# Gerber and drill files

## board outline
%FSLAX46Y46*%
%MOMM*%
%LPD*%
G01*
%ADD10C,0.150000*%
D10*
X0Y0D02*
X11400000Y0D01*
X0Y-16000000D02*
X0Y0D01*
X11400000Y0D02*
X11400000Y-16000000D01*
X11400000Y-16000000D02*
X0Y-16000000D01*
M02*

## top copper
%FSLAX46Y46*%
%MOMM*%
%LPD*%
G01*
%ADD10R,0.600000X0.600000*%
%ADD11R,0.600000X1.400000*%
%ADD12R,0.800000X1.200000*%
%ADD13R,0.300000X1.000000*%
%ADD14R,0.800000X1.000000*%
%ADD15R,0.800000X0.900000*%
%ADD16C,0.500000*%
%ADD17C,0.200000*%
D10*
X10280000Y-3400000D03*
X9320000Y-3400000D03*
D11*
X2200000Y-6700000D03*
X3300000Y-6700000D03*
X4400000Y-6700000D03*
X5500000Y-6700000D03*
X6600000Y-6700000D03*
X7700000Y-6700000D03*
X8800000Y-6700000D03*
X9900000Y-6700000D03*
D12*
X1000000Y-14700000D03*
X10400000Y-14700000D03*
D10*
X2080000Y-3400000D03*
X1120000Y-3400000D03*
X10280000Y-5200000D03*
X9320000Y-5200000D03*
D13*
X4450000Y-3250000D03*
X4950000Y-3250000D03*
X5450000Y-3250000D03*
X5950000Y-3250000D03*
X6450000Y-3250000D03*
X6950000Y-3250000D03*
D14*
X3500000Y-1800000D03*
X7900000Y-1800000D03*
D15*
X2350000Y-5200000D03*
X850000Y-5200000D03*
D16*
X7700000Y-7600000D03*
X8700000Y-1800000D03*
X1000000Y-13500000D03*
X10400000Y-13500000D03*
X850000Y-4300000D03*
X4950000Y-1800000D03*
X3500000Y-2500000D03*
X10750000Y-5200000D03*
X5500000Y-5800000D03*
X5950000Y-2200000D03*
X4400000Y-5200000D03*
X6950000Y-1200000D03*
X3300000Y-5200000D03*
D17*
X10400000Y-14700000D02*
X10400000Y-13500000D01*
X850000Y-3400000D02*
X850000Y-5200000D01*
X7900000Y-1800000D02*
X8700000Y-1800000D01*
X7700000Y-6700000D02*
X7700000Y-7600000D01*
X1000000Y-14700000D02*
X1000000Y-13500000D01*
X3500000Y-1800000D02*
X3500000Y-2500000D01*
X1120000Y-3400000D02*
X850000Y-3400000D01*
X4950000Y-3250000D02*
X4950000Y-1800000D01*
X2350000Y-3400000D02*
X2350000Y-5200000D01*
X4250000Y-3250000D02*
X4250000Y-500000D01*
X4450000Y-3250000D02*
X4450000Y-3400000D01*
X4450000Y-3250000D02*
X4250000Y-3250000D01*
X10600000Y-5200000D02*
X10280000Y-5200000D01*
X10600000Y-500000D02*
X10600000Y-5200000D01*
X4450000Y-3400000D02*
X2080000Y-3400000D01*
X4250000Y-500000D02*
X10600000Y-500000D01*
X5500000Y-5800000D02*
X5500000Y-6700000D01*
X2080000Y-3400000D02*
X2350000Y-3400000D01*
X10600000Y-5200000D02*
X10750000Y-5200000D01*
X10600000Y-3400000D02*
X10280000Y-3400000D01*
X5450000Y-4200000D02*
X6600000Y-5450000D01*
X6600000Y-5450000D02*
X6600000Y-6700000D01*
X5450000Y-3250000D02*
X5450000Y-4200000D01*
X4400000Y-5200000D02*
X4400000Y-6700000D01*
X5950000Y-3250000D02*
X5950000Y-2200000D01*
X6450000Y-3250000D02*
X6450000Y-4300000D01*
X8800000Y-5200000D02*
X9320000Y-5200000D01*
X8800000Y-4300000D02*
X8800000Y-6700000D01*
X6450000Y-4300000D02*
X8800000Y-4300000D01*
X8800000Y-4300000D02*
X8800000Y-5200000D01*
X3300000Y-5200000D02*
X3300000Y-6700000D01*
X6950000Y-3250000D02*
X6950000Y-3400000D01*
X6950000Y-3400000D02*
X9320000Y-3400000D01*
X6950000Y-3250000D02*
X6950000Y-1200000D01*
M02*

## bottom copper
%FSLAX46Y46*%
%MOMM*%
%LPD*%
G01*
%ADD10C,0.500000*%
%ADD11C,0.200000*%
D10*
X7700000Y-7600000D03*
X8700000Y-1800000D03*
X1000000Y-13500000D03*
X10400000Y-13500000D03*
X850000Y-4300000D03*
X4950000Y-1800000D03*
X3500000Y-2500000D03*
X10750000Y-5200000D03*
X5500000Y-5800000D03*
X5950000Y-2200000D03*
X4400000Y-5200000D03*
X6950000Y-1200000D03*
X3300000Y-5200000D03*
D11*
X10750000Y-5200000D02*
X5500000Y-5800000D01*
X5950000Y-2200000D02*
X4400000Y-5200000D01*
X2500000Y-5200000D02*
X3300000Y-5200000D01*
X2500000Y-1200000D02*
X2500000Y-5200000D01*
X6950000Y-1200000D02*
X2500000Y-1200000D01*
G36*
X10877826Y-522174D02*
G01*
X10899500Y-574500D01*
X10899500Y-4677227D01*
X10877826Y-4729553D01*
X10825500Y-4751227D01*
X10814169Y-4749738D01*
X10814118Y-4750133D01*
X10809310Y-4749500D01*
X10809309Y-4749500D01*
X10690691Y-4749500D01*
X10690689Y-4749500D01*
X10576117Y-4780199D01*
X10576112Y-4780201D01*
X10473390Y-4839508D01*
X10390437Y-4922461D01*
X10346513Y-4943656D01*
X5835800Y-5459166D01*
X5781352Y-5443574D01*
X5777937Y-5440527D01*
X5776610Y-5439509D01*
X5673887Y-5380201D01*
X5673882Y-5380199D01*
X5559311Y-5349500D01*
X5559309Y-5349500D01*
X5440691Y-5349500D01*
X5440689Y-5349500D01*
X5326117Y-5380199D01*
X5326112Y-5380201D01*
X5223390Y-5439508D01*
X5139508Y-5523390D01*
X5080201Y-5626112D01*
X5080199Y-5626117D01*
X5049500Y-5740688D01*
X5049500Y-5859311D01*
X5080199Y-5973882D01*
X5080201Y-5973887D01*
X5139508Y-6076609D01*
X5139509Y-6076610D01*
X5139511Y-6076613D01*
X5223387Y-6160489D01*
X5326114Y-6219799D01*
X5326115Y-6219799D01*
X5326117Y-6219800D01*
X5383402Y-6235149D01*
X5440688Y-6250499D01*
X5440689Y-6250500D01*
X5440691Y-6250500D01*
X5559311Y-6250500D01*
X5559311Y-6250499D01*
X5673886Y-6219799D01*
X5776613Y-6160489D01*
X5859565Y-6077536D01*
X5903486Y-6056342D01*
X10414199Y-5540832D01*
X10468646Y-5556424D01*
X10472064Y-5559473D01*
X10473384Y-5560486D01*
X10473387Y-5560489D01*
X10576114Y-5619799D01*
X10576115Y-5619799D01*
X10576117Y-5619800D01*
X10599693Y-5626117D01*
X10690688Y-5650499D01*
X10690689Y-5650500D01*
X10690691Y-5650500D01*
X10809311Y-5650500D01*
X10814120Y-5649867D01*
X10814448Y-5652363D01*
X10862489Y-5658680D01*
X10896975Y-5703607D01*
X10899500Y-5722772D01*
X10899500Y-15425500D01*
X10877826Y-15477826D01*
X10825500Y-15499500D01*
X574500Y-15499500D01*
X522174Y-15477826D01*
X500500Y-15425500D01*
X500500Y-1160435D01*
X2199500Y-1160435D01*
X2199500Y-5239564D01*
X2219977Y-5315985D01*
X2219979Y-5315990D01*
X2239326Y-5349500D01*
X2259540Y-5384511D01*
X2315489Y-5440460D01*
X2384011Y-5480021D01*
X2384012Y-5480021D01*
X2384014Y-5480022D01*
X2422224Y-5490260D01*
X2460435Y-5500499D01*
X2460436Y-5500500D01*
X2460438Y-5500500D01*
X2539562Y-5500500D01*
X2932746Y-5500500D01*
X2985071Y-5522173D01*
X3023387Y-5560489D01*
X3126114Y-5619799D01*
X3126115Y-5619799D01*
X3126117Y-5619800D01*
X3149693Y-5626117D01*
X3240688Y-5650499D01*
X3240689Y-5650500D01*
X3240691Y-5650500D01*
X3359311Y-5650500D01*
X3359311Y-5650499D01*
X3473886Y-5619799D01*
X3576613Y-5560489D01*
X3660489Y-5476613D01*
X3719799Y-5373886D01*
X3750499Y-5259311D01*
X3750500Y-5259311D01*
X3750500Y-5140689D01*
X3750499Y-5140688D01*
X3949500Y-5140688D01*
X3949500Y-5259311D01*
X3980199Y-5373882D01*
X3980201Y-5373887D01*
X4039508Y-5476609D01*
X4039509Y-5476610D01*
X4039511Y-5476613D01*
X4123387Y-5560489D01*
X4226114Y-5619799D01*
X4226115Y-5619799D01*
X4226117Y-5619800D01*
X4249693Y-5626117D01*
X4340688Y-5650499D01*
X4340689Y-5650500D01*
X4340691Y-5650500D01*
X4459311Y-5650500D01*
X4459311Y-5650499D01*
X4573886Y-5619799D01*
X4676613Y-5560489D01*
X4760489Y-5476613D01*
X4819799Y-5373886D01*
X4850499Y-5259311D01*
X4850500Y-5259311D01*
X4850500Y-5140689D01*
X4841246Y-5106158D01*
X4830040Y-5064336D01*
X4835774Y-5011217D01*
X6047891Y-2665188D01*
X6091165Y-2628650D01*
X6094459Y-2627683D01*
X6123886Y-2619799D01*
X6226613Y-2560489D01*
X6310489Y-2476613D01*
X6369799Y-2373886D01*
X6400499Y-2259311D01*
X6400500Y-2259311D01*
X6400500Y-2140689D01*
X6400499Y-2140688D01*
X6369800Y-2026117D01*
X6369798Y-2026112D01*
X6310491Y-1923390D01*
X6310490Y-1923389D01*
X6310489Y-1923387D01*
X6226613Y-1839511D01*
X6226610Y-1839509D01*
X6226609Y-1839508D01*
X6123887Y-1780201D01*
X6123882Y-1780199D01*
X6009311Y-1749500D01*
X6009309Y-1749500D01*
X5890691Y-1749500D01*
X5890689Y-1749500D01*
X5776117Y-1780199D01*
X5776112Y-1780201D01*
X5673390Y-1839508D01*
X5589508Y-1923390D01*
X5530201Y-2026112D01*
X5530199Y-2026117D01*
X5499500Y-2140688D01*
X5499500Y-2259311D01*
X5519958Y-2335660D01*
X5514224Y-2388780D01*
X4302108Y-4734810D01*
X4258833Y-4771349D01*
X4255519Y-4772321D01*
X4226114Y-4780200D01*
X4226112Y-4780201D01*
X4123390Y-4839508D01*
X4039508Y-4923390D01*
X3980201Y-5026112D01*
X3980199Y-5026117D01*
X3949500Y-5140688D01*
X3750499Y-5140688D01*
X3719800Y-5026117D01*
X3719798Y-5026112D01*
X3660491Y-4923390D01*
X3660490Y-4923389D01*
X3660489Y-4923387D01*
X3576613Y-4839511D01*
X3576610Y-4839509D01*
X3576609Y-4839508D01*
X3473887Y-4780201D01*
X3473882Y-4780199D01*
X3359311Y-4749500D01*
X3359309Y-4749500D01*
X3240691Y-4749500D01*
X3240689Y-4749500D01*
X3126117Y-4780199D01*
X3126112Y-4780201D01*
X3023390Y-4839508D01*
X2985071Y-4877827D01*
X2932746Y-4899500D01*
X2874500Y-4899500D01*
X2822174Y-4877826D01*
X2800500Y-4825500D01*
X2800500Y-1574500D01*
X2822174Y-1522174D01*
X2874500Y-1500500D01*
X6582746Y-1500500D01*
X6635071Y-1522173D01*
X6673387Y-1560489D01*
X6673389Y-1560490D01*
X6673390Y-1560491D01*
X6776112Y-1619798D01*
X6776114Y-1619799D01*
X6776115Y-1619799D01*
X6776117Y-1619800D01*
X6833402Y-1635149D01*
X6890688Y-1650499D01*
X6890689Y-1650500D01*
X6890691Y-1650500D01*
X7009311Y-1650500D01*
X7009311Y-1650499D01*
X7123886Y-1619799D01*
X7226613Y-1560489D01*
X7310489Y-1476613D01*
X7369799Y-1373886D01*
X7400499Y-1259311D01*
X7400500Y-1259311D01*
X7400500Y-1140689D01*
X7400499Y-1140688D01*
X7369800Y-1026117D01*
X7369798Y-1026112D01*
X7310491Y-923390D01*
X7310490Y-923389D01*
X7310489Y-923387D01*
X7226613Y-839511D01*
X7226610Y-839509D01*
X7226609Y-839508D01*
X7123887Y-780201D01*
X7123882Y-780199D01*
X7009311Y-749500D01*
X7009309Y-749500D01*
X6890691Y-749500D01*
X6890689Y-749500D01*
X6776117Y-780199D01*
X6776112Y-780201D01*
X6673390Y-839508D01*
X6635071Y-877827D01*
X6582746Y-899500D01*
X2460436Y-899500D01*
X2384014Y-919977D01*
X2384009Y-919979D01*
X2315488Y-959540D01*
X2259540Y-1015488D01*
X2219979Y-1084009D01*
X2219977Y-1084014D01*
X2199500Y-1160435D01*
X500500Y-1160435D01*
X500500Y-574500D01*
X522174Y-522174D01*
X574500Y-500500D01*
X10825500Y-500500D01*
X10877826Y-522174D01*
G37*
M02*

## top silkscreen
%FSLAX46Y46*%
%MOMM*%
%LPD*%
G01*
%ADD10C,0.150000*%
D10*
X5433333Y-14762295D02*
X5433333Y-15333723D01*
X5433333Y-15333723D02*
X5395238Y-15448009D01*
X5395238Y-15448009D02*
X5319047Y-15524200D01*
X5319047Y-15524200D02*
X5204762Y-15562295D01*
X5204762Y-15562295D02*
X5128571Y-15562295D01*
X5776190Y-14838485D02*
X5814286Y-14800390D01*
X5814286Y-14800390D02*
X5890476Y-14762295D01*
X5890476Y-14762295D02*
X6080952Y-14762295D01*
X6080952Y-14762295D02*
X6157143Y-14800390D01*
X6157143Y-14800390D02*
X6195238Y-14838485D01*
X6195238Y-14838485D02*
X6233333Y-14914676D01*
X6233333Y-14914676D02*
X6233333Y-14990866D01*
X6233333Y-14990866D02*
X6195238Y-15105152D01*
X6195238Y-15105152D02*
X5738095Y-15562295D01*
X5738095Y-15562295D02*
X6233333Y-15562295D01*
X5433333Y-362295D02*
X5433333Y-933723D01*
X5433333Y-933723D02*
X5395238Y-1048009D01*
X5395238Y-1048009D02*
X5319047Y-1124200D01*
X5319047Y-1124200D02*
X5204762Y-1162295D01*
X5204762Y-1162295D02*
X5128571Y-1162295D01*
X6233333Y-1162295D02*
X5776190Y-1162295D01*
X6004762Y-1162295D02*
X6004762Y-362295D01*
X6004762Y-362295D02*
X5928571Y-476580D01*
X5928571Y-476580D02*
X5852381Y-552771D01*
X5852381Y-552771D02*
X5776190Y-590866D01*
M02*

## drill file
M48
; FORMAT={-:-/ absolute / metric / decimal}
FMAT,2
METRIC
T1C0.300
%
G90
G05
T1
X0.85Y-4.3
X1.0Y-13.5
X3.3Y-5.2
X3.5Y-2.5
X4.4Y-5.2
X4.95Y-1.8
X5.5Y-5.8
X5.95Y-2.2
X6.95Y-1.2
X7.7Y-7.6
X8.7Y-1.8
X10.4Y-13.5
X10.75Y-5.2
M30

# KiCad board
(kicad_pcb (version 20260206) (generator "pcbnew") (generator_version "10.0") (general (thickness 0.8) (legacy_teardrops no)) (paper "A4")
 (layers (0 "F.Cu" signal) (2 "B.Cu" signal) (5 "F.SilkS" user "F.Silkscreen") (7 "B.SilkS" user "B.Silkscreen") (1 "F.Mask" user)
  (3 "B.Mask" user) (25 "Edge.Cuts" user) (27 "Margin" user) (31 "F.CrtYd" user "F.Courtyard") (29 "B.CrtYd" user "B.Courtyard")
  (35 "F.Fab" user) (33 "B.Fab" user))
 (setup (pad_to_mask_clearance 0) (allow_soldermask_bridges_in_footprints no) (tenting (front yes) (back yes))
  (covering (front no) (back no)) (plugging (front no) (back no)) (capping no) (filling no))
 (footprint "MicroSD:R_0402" (layer "F.Cu") (at 9.8 3.4)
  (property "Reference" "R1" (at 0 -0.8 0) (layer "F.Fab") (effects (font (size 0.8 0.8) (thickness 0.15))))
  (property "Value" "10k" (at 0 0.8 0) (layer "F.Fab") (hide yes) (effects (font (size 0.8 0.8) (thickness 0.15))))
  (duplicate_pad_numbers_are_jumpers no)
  (pad "1" smd rect (at 0.48 0) (size 0.6 0.6) (layers "F.Cu" "F.Mask" "F.Paste") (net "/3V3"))
  (pad "2" smd rect (at -0.48 0) (size 0.6 0.6) (layers "F.Cu" "F.Mask" "F.Paste") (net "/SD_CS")))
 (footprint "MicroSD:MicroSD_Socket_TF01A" (layer "F.Cu") (at 5.7 11.2)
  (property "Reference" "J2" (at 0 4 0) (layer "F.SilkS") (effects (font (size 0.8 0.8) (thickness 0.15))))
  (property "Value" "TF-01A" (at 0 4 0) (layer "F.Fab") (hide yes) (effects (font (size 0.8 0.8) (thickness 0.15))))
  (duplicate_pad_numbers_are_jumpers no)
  (pad "1" smd rect (at -3.5 -4.5) (size 0.6 1.4) (layers "F.Cu" "F.Mask" "F.Paste") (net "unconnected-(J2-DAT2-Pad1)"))
  (pad "2" smd rect (at -2.4 -4.5) (size 0.6 1.4) (layers "F.Cu" "F.Mask" "F.Paste") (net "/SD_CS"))
  (pad "3" smd rect (at -1.3 -4.5) (size 0.6 1.4) (layers "F.Cu" "F.Mask" "F.Paste") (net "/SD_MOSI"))
  (pad "4" smd rect (at -0.2 -4.5) (size 0.6 1.4) (layers "F.Cu" "F.Mask" "F.Paste") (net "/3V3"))
  (pad "5" smd rect (at 0.9 -4.5) (size 0.6 1.4) (layers "F.Cu" "F.Mask" "F.Paste") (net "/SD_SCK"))
  (pad "6" smd rect (at 2 -4.5) (size 0.6 1.4) (layers "F.Cu" "F.Mask" "F.Paste") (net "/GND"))
  (pad "7" smd rect (at 3.1 -4.5) (size 0.6 1.4) (layers "F.Cu" "F.Mask" "F.Paste") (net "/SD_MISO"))
  (pad "8" smd rect (at 4.2 -4.5) (size 0.6 1.4) (layers "F.Cu" "F.Mask" "F.Paste") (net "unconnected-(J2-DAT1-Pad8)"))
  (pad "9" smd rect (at -4.7 3.5) (size 0.8 1.2) (layers "F.Cu" "F.Mask" "F.Paste") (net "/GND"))
  (pad "10" smd rect (at 4.7 3.5) (size 0.8 1.2) (layers "F.Cu" "F.Mask" "F.Paste") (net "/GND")))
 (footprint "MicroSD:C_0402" (layer "F.Cu") (at 1.6 3.4)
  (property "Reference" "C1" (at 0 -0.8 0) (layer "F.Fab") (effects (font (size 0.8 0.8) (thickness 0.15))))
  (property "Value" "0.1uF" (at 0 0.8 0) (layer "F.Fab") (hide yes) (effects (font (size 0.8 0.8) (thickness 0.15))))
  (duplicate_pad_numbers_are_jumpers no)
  (pad "1" smd rect (at 0.48 0) (size 0.6 0.6) (layers "F.Cu" "F.Mask" "F.Paste") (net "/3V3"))
  (pad "2" smd rect (at -0.48 0) (size 0.6 0.6) (layers "F.Cu" "F.Mask" "F.Paste") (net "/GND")))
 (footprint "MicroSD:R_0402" (layer "F.Cu") (at 9.8 5.2)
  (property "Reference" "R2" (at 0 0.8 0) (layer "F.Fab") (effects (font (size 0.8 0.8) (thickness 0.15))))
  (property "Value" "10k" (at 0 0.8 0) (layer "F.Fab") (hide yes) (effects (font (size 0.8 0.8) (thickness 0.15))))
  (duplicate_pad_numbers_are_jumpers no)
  (pad "1" smd rect (at 0.48 0) (size 0.6 0.6) (layers "F.Cu" "F.Mask" "F.Paste") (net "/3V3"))
  (pad "2" smd rect (at -0.48 0) (size 0.6 0.6) (layers "F.Cu" "F.Mask" "F.Paste") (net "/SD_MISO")))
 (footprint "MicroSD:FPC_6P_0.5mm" (layer "F.Cu") (at 5.7 2)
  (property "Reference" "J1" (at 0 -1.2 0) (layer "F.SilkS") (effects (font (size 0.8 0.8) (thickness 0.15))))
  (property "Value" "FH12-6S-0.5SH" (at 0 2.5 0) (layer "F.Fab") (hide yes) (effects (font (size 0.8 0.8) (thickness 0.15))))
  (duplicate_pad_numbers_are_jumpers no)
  (pad "1" smd rect (at -1.25 1.25) (size 0.3 1) (layers "F.Cu" "F.Mask" "F.Paste") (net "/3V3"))
  (pad "2" smd rect (at -0.75 1.25) (size 0.3 1) (layers "F.Cu" "F.Mask" "F.Paste") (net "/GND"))
  (pad "3" smd rect (at -0.25 1.25) (size 0.3 1) (layers "F.Cu" "F.Mask" "F.Paste") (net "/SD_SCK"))
  (pad "4" smd rect (at 0.25 1.25) (size 0.3 1) (layers "F.Cu" "F.Mask" "F.Paste") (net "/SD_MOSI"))
  (pad "5" smd rect (at 0.75 1.25) (size 0.3 1) (layers "F.Cu" "F.Mask" "F.Paste") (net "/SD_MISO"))
  (pad "6" smd rect (at 1.25 1.25) (size 0.3 1) (layers "F.Cu" "F.Mask" "F.Paste") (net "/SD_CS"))
  (pad "MP1" smd rect (at -2.2 -0.2) (size 0.8 1) (layers "F.Cu" "F.Mask" "F.Paste") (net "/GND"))
  (pad "MP2" smd rect (at 2.2 -0.2) (size 0.8 1) (layers "F.Cu" "F.Mask" "F.Paste") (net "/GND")))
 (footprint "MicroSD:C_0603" (layer "F.Cu") (at 1.6 5.2)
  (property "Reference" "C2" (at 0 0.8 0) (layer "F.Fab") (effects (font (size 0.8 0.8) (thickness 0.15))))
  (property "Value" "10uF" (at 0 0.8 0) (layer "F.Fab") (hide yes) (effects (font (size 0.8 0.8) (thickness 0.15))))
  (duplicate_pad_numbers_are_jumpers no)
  (pad "1" smd rect (at 0.75 0) (size 0.8 0.9) (layers "F.Cu" "F.Mask" "F.Paste") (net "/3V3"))
  (pad "2" smd rect (at -0.75 0) (size 0.8 0.9) (layers "F.Cu" "F.Mask" "F.Paste") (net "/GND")))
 (gr_line (start 0 0) (end 11.4 0) (stroke (width 0.15) (type solid)) (layer "Edge.Cuts"))
 (gr_line (start 0 16) (end 0 0) (stroke (width 0.15) (type solid)) (layer "Edge.Cuts"))
 (gr_line (start 11.4 0) (end 11.4 16) (stroke (width 0.15) (type solid)) (layer "Edge.Cuts"))
 (gr_line (start 11.4 16) (end 0 16) (stroke (width 0.15) (type solid)) (layer "Edge.Cuts"))
 (segment (start 10.4 14.7) (end 10.4 13.5) (width 0.2) (layer "F.Cu") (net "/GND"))
 (segment (start 0.85 3.4) (end 0.85 5.2) (width 0.2) (layer "F.Cu") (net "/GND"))
 (segment (start 7.9 1.8) (end 8.7 1.8) (width 0.2) (layer "F.Cu") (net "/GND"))
 (segment (start 7.7 6.7) (end 7.7 7.6) (width 0.2) (layer "F.Cu") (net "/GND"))
 (segment (start 1 14.7) (end 1 13.5) (width 0.2) (layer "F.Cu") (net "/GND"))
 (segment (start 3.5 1.8) (end 3.5 2.5) (width 0.2) (layer "F.Cu") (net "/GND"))
 (segment (start 1.12 3.4) (end 0.85 3.4) (width 0.2) (layer "F.Cu") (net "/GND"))
 (segment (start 4.95 3.25) (end 4.95 1.8) (width 0.2) (layer "F.Cu") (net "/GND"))
 (via (at 7.7 7.6) (size 0.5) (drill 0.3) (layers "F.Cu" "B.Cu") (capping no) (covering (front no) (back no))
  (plugging (front no) (back no)) (filling no) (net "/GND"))
 (via (at 8.7 1.8) (size 0.5) (drill 0.3) (layers "F.Cu" "B.Cu") (capping no) (covering (front no) (back no))
  (plugging (front no) (back no)) (filling no) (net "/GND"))
 (via (at 1 13.5) (size 0.5) (drill 0.3) (layers "F.Cu" "B.Cu") (capping no) (covering (front no) (back no)) (plugging (front no) (back no))
  (filling no) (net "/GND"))
 (via (at 10.4 13.5) (size 0.5) (drill 0.3) (layers "F.Cu" "B.Cu") (capping no) (covering (front no) (back no))
  (plugging (front no) (back no)) (filling no) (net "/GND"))
 (via (at 0.85 4.3) (size 0.5) (drill 0.3) (layers "F.Cu" "B.Cu") (capping no) (covering (front no) (back no))
  (plugging (front no) (back no)) (filling no) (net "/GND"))
 (via (at 4.95 1.8) (size 0.5) (drill 0.3) (layers "F.Cu" "B.Cu") (capping no) (covering (front no) (back no))
  (plugging (front no) (back no)) (filling no) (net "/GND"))
 (via (at 3.5 2.5) (size 0.5) (drill 0.3) (layers "F.Cu" "B.Cu") (capping no) (covering (front no) (back no))
  (plugging (front no) (back no)) (filling no) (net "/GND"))
 (segment (start 2.35 3.4) (end 2.35 5.2) (width 0.2) (layer "F.Cu") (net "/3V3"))
 (segment (start 4.25 3.25) (end 4.25 0.5) (width 0.2) (layer "F.Cu") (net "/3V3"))
 (segment (start 4.45 3.25) (end 4.45 3.4) (width 0.2) (layer "F.Cu") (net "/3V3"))
 (segment (start 4.45 3.25) (end 4.25 3.25) (width 0.2) (layer "F.Cu") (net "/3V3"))
 (segment (start 10.6 5.2) (end 10.28 5.2) (width 0.2) (layer "F.Cu") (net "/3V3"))
 (segment (start 10.6 0.5) (end 10.6 5.2) (width 0.2) (layer "F.Cu") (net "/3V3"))
 (segment (start 4.45 3.4) (end 2.08 3.4) (width 0.2) (layer "F.Cu") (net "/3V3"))
 (segment (start 4.25 0.5) (end 10.6 0.5) (width 0.2) (layer "F.Cu") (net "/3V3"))
 (segment (start 5.5 5.8) (end 5.5 6.7) (width 0.2) (layer "F.Cu") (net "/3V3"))
 (segment (start 2.08 3.4) (end 2.35 3.4) (width 0.2) (layer "F.Cu") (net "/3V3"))
 (segment (start 10.6 5.2) (end 10.75 5.2) (width 0.2) (layer "F.Cu") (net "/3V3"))
 (segment (start 10.6 3.4) (end 10.28 3.4) (width 0.2) (layer "F.Cu") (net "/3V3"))
 (via (at 10.75 5.2) (size 0.5) (drill 0.3) (layers "F.Cu" "B.Cu") (capping no) (covering (front no) (back no))
  (plugging (front no) (back no)) (filling no) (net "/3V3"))
 (via (at 5.5 5.8) (size 0.5) (drill 0.3) (layers "F.Cu" "B.Cu") (capping no) (covering (front no) (back no))
  (plugging (front no) (back no)) (filling no) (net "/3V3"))
 (segment (start 10.75 5.2) (end 5.5 5.8) (width 0.2) (layer "B.Cu") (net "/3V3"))
 (segment (start 5.45 4.2) (end 6.6 5.45) (width 0.2) (layer "F.Cu") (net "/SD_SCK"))
 (segment (start 6.6 5.45) (end 6.6 6.7) (width 0.2) (layer "F.Cu") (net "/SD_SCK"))
 (segment (start 5.45 3.25) (end 5.45 4.2) (width 0.2) (layer "F.Cu") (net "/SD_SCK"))
 (segment (start 4.4 5.2) (end 4.4 6.7) (width 0.2) (layer "F.Cu") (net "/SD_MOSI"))
 (segment (start 5.95 3.25) (end 5.95 2.2) (width 0.2) (layer "F.Cu") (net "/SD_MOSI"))
 (via (at 5.95 2.2) (size 0.5) (drill 0.3) (layers "F.Cu" "B.Cu") (capping no) (covering (front no) (back no))
  (plugging (front no) (back no)) (filling no) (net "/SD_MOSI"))
 (via (at 4.4 5.2) (size 0.5) (drill 0.3) (layers "F.Cu" "B.Cu") (capping no) (covering (front no) (back no))
  (plugging (front no) (back no)) (filling no) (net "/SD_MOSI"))
 (segment (start 5.95 2.2) (end 4.4 5.2) (width 0.2) (layer "B.Cu") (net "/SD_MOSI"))
 (segment (start 6.45 3.25) (end 6.45 4.3) (width 0.2) (layer "F.Cu") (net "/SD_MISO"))
 (segment (start 8.8 5.2) (end 9.32 5.2) (width 0.2) (layer "F.Cu") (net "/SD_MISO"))
 (segment (start 8.8 4.3) (end 8.8 6.7) (width 0.2) (layer "F.Cu") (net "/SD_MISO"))
 (segment (start 6.45 4.3) (end 8.8 4.3) (width 0.2) (layer "F.Cu") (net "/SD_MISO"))
 (segment (start 8.8 4.3) (end 8.8 5.2) (width 0.2) (layer "F.Cu") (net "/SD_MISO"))
 (segment (start 3.3 5.2) (end 3.3 6.7) (width 0.2) (layer "F.Cu") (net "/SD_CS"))
 (segment (start 6.95 3.25) (end 6.95 3.4) (width 0.2) (layer "F.Cu") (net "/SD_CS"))
 (segment (start 6.95 3.4) (end 9.32 3.4) (width 0.2) (layer "F.Cu") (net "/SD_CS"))
 (segment (start 6.95 3.25) (end 6.95 1.2) (width 0.2) (layer "F.Cu") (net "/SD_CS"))
 (via (at 6.95 1.2) (size 0.5) (drill 0.3) (layers "F.Cu" "B.Cu") (capping no) (covering (front no) (back no))
  (plugging (front no) (back no)) (filling no) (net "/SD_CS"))
 (via (at 3.3 5.2) (size 0.5) (drill 0.3) (layers "F.Cu" "B.Cu") (capping no) (covering (front no) (back no))
  (plugging (front no) (back no)) (filling no) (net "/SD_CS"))
 (segment (start 2.5 5.2) (end 3.3 5.2) (width 0.2) (layer "B.Cu") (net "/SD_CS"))
 (segment (start 2.5 1.2) (end 2.5 5.2) (width 0.2) (layer "B.Cu") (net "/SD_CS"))
 (segment (start 6.95 1.2) (end 2.5 1.2) (width 0.2) (layer "B.Cu") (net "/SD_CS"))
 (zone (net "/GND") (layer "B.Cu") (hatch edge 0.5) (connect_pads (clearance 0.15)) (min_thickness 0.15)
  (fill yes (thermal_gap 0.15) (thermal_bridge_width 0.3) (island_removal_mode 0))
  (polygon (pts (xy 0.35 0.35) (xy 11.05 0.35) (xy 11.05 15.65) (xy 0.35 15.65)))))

